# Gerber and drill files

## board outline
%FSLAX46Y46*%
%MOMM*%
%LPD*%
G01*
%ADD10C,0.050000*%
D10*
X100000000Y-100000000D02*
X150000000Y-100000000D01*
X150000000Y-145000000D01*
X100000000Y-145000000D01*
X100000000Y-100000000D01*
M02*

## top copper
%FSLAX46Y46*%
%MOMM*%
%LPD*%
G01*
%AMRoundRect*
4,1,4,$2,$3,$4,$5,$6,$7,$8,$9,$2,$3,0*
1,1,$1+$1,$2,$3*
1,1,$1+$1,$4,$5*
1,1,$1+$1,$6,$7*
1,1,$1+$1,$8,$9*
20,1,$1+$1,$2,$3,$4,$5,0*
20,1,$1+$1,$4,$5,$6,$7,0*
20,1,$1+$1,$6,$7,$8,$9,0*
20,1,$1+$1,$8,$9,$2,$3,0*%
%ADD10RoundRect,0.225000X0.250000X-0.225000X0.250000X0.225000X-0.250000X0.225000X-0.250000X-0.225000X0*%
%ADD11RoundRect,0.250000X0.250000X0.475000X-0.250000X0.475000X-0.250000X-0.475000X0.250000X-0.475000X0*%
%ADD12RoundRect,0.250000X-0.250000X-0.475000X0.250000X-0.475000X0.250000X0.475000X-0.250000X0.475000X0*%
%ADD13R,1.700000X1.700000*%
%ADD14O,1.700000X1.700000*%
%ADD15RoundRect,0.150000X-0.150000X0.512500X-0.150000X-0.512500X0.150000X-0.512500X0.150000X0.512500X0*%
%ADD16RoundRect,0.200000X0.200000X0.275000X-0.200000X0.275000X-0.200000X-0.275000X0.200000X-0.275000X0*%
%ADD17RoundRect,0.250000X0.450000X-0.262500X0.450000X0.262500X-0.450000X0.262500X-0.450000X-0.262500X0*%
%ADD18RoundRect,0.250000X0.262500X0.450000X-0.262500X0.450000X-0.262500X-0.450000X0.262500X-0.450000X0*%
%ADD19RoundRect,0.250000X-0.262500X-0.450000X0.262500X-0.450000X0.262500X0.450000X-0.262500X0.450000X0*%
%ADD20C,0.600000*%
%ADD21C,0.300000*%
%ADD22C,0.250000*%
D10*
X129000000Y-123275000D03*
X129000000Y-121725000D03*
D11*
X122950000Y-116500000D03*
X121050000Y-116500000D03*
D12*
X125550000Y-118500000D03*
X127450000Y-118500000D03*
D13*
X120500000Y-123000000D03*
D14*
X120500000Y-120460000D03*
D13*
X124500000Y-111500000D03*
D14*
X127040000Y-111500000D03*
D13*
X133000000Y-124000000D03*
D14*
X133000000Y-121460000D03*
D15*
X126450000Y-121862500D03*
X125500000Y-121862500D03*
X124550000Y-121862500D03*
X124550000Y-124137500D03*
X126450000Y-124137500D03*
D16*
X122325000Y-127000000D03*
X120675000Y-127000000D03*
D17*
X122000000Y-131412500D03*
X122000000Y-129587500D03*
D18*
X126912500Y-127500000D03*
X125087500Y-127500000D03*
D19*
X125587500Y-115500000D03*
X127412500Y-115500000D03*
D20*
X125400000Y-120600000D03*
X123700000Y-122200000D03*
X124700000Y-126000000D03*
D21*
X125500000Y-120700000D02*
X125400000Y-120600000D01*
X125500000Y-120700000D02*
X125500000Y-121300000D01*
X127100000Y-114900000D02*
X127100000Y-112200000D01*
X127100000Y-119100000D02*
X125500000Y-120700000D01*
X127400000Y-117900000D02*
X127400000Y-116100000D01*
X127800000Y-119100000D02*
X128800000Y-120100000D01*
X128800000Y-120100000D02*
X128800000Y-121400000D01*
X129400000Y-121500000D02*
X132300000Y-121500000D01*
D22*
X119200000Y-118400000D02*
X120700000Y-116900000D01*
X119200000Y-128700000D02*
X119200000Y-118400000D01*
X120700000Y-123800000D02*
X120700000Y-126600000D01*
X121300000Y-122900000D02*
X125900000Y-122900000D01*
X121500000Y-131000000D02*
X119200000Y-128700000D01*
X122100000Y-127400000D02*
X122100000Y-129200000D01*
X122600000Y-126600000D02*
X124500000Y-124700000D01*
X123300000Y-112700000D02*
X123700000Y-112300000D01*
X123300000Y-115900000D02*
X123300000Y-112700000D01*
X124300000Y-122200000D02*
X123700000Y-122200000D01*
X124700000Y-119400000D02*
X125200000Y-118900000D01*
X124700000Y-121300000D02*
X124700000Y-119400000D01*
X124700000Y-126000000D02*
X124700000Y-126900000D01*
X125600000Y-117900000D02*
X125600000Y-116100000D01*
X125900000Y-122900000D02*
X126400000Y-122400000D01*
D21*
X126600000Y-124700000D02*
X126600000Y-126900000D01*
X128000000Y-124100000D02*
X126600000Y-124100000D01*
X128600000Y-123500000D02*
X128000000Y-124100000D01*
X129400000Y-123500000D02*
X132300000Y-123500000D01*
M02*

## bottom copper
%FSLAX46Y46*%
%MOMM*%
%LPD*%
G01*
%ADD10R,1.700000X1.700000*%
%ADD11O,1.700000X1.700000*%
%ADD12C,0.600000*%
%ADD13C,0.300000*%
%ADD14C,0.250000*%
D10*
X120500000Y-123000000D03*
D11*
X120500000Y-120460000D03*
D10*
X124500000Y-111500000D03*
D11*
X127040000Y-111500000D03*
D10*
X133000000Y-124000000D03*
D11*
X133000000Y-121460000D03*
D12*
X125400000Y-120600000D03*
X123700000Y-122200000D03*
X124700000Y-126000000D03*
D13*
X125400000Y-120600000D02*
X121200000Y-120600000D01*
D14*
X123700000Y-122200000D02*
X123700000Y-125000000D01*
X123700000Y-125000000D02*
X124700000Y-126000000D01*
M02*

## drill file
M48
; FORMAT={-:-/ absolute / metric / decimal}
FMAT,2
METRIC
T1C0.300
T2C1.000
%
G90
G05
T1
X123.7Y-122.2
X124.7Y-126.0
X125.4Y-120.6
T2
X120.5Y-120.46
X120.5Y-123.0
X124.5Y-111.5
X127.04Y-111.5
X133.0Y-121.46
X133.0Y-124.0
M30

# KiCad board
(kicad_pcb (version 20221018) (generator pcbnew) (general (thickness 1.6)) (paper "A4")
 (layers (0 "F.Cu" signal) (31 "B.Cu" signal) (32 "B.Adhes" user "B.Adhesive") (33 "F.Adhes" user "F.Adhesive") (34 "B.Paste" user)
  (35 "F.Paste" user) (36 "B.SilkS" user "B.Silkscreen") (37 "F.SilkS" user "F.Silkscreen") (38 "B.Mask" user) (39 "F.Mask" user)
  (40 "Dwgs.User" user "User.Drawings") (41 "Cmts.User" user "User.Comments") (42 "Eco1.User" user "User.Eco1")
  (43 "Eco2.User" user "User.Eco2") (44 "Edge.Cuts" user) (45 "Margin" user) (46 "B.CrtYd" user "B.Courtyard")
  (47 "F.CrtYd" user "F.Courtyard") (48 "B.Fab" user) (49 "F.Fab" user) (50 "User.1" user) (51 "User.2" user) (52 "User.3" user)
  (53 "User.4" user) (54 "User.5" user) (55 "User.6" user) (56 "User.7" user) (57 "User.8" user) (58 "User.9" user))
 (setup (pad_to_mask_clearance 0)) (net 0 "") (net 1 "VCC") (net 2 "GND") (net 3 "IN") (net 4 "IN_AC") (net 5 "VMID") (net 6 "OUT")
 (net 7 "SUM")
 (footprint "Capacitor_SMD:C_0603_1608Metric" (layer "F.Cu") (at 129 122.5 90)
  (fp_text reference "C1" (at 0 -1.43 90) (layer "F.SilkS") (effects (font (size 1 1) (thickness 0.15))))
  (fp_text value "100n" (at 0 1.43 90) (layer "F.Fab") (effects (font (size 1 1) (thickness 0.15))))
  (pad "1" smd roundrect (at -0.775 0 90) (size 0.9 0.95) (layers "F.Cu" "F.Paste" "F.Mask") (roundrect_rratio 0.25) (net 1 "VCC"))
  (pad "2" smd roundrect (at 0.775 0 90) (size 0.9 0.95) (layers "F.Cu" "F.Paste" "F.Mask") (roundrect_rratio 0.25) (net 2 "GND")))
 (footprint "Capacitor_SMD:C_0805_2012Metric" (layer "F.Cu") (at 122 116.5 180)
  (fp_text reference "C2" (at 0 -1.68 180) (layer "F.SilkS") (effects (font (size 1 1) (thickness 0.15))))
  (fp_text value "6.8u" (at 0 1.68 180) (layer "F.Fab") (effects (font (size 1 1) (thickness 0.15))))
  (pad "1" smd roundrect (at -0.95 0 180) (size 1 1.45) (layers "F.Cu" "F.Paste" "F.Mask") (roundrect_rratio 0.25) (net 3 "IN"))
  (pad "2" smd roundrect (at 0.95 0 180) (size 1 1.45) (layers "F.Cu" "F.Paste" "F.Mask") (roundrect_rratio 0.25) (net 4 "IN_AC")))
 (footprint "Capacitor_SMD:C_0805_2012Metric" (layer "F.Cu") (at 126.5 118.5)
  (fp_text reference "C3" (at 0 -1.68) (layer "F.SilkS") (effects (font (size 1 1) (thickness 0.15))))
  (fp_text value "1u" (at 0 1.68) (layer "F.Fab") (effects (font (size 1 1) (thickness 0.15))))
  (pad "1" smd roundrect (at -0.95 0) (size 1 1.45) (layers "F.Cu" "F.Paste" "F.Mask") (roundrect_rratio 0.25) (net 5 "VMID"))
  (pad "2" smd roundrect (at 0.95 0) (size 1 1.45) (layers "F.Cu" "F.Paste" "F.Mask") (roundrect_rratio 0.25) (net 2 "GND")))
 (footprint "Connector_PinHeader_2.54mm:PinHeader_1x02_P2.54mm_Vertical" (layer "F.Cu") (at 120.5 123 180)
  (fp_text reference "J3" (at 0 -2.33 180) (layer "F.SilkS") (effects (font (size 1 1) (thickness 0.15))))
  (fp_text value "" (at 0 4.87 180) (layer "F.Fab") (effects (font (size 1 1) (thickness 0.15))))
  (pad "1" thru_hole rect (at 0 0 180) (size 1.7 1.7) (drill 1) (layers "*.Cu" "*.Mask") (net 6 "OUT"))
  (pad "2" thru_hole oval (at 0 2.54 180) (size 1.7 1.7) (drill 1) (layers "*.Cu" "*.Mask") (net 2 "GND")))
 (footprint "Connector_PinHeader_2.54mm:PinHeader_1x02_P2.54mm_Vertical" (layer "F.Cu") (at 124.5 111.5 90)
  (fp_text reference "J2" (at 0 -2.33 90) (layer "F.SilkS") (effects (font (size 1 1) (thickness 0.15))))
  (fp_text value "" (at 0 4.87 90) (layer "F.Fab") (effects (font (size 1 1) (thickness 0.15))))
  (pad "1" thru_hole rect (at 0 0 90) (size 1.7 1.7) (drill 1) (layers "*.Cu" "*.Mask") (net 3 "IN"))
  (pad "2" thru_hole oval (at 0 2.54 90) (size 1.7 1.7) (drill 1) (layers "*.Cu" "*.Mask") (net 2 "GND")))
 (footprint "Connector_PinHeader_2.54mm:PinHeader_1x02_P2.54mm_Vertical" (layer "F.Cu") (at 133 124 180)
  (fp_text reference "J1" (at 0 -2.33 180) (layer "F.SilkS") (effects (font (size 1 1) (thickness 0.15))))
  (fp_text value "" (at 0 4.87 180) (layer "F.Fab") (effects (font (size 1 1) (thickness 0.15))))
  (pad "1" thru_hole rect (at 0 0 180) (size 1.7 1.7) (drill 1) (layers "*.Cu" "*.Mask") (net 1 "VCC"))
  (pad "2" thru_hole oval (at 0 2.54 180) (size 1.7 1.7) (drill 1) (layers "*.Cu" "*.Mask") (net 2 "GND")))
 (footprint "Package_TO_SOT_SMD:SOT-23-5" (layer "F.Cu") (at 125.5 123 -90)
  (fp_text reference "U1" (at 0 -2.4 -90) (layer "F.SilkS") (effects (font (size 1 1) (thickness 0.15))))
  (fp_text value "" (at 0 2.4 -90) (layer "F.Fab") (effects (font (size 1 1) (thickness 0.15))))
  (pad "1" smd roundrect (at -1.1375 -0.95 270) (size 1.325 0.6) (layers "F.Cu" "F.Paste" "F.Mask") (roundrect_rratio 0.25) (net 6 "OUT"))
  (pad "2" smd roundrect (at -1.1375 0 270) (size 1.325 0.6) (layers "F.Cu" "F.Paste" "F.Mask") (roundrect_rratio 0.25) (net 2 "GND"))
  (pad "3" smd roundrect (at -1.1375 0.95 270) (size 1.325 0.6) (layers "F.Cu" "F.Paste" "F.Mask") (roundrect_rratio 0.25) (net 5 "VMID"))
  (pad "4" smd roundrect (at 1.1375 0.95 270) (size 1.325 0.6) (layers "F.Cu" "F.Paste" "F.Mask") (roundrect_rratio 0.25) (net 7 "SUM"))
  (pad "5" smd roundrect (at 1.1375 -0.95 270) (size 1.325 0.6) (layers "F.Cu" "F.Paste" "F.Mask") (roundrect_rratio 0.25) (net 1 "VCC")))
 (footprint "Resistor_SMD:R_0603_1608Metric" (layer "F.Cu") (at 121.5 127 180)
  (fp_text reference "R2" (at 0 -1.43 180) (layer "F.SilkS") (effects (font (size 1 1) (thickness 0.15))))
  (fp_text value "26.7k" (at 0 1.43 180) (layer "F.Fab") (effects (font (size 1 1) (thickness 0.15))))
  (pad "1" smd roundrect (at -0.825 0 180) (size 0.8 0.95) (layers "F.Cu" "F.Paste" "F.Mask") (roundrect_rratio 0.25) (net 7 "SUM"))
  (pad "2" smd roundrect (at 0.825 0 180) (size 0.8 0.95) (layers "F.Cu" "F.Paste" "F.Mask") (roundrect_rratio 0.25) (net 6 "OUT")))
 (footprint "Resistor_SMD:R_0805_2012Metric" (layer "F.Cu") (at 122 130.5 90)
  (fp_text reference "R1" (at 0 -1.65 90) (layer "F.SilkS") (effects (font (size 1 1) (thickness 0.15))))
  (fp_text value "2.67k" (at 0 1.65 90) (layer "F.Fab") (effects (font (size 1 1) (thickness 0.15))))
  (pad "1" smd roundrect (at -0.9125 0 90) (size 1.025 1.4) (layers "F.Cu" "F.Paste" "F.Mask") (roundrect_rratio 0.243902) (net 4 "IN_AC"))
  (pad "2" smd roundrect (at 0.9125 0 90) (size 1.025 1.4) (layers "F.Cu" "F.Paste" "F.Mask") (roundrect_rratio 0.243902) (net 7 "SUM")))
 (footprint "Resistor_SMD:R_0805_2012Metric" (layer "F.Cu") (at 126 127.5 180)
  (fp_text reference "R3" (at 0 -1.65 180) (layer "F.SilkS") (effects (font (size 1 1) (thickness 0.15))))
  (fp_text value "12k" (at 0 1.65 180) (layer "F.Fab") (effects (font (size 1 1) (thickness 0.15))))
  (pad "1" smd roundrect (at -0.9125 0 180) (size 1.025 1.4) (layers "F.Cu" "F.Paste" "F.Mask") (roundrect_rratio 0.243902) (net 1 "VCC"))
  (pad "2" smd roundrect (at 0.9125 0 180) (size 1.025 1.4) (layers "F.Cu" "F.Paste" "F.Mask") (roundrect_rratio 0.243902) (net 5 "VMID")))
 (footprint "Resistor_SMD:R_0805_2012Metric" (layer "F.Cu") (at 126.5 115.5)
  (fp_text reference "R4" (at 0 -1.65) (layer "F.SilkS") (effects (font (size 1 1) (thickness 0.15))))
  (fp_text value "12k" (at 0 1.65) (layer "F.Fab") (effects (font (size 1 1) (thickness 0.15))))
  (pad "1" smd roundrect (at -0.9125 0) (size 1.025 1.4) (layers "F.Cu" "F.Paste" "F.Mask") (roundrect_rratio 0.243902) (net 5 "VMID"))
  (pad "2" smd roundrect (at 0.9125 0) (size 1.025 1.4) (layers "F.Cu" "F.Paste" "F.Mask") (roundrect_rratio 0.243902) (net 2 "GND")))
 (gr_rect (start 100 100) (end 150 145) (stroke (width 0.05) (type default)) (fill none) (layer "Edge.Cuts"))
 (segment (start 125.5 120.7) (end 125.4 120.6) (width 0.3) (layer "F.Cu") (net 2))
 (segment (start 125.5 120.7) (end 125.5 121.3) (width 0.3) (layer "F.Cu") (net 2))
 (segment (start 127.1 114.9) (end 127.1 112.2) (width 0.3) (layer "F.Cu") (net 2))
 (segment (start 127.1 119.1) (end 125.5 120.7) (width 0.3) (layer "F.Cu") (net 2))
 (segment (start 127.4 117.9) (end 127.4 116.1) (width 0.3) (layer "F.Cu") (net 2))
 (segment (start 127.8 119.1) (end 128.8 120.1) (width 0.3) (layer "F.Cu") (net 2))
 (segment (start 128.8 120.1) (end 128.8 121.4) (width 0.3) (layer "F.Cu") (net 2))
 (segment (start 129.4 121.5) (end 132.3 121.5) (width 0.3) (layer "F.Cu") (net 2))
 (via (at 125.4 120.6) (size 0.6) (drill 0.3) (layers "F.Cu" "B.Cu") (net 2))
 (segment (start 119.2 118.4) (end 120.7 116.9) (width 0.25) (layer "F.Cu") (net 4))
 (segment (start 119.2 128.7) (end 119.2 118.4) (width 0.25) (layer "F.Cu") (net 4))
 (segment (start 120.7 123.8) (end 120.7 126.6) (width 0.25) (layer "F.Cu") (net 6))
 (segment (start 121.3 122.9) (end 125.9 122.9) (width 0.25) (layer "F.Cu") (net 6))
 (segment (start 121.5 131) (end 119.2 128.7) (width 0.25) (layer "F.Cu") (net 4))
 (segment (start 122.1 127.4) (end 122.1 129.2) (width 0.25) (layer "F.Cu") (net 7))
 (segment (start 122.6 126.6) (end 124.5 124.7) (width 0.25) (layer "F.Cu") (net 7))
 (segment (start 123.3 112.7) (end 123.7 112.3) (width 0.25) (layer "F.Cu") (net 3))
 (segment (start 123.3 115.9) (end 123.3 112.7) (width 0.25) (layer "F.Cu") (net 3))
 (segment (start 124.3 122.2) (end 123.7 122.2) (width 0.25) (layer "F.Cu") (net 5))
 (segment (start 124.7 119.4) (end 125.2 118.9) (width 0.25) (layer "F.Cu") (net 5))
 (segment (start 124.7 121.3) (end 124.7 119.4) (width 0.25) (layer "F.Cu") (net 5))
 (segment (start 124.7 126) (end 124.7 126.9) (width 0.25) (layer "F.Cu") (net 5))
 (segment (start 125.4 120.6) (end 121.2 120.6) (width 0.3) (layer "B.Cu") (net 2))
 (segment (start 125.6 117.9) (end 125.6 116.1) (width 0.25) (layer "F.Cu") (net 5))
 (segment (start 125.9 122.9) (end 126.4 122.4) (width 0.25) (layer "F.Cu") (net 6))
 (segment (start 126.6 124.7) (end 126.6 126.9) (width 0.3) (layer "F.Cu") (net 1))
 (segment (start 128 124.1) (end 126.6 124.1) (width 0.3) (layer "F.Cu") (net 1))
 (segment (start 128.6 123.5) (end 128 124.1) (width 0.3) (layer "F.Cu") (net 1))
 (segment (start 129.4 123.5) (end 132.3 123.5) (width 0.3) (layer "F.Cu") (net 1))
 (via (at 123.7 122.2) (size 0.6) (drill 0.3) (layers "F.Cu" "B.Cu") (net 5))
 (via (at 124.7 126) (size 0.6) (drill 0.3) (layers "F.Cu" "B.Cu") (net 5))
 (segment (start 123.7 122.2) (end 123.7 125) (width 0.25) (layer "B.Cu") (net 5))
 (segment (start 123.7 125) (end 124.7 126) (width 0.25) (layer "B.Cu") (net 5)))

